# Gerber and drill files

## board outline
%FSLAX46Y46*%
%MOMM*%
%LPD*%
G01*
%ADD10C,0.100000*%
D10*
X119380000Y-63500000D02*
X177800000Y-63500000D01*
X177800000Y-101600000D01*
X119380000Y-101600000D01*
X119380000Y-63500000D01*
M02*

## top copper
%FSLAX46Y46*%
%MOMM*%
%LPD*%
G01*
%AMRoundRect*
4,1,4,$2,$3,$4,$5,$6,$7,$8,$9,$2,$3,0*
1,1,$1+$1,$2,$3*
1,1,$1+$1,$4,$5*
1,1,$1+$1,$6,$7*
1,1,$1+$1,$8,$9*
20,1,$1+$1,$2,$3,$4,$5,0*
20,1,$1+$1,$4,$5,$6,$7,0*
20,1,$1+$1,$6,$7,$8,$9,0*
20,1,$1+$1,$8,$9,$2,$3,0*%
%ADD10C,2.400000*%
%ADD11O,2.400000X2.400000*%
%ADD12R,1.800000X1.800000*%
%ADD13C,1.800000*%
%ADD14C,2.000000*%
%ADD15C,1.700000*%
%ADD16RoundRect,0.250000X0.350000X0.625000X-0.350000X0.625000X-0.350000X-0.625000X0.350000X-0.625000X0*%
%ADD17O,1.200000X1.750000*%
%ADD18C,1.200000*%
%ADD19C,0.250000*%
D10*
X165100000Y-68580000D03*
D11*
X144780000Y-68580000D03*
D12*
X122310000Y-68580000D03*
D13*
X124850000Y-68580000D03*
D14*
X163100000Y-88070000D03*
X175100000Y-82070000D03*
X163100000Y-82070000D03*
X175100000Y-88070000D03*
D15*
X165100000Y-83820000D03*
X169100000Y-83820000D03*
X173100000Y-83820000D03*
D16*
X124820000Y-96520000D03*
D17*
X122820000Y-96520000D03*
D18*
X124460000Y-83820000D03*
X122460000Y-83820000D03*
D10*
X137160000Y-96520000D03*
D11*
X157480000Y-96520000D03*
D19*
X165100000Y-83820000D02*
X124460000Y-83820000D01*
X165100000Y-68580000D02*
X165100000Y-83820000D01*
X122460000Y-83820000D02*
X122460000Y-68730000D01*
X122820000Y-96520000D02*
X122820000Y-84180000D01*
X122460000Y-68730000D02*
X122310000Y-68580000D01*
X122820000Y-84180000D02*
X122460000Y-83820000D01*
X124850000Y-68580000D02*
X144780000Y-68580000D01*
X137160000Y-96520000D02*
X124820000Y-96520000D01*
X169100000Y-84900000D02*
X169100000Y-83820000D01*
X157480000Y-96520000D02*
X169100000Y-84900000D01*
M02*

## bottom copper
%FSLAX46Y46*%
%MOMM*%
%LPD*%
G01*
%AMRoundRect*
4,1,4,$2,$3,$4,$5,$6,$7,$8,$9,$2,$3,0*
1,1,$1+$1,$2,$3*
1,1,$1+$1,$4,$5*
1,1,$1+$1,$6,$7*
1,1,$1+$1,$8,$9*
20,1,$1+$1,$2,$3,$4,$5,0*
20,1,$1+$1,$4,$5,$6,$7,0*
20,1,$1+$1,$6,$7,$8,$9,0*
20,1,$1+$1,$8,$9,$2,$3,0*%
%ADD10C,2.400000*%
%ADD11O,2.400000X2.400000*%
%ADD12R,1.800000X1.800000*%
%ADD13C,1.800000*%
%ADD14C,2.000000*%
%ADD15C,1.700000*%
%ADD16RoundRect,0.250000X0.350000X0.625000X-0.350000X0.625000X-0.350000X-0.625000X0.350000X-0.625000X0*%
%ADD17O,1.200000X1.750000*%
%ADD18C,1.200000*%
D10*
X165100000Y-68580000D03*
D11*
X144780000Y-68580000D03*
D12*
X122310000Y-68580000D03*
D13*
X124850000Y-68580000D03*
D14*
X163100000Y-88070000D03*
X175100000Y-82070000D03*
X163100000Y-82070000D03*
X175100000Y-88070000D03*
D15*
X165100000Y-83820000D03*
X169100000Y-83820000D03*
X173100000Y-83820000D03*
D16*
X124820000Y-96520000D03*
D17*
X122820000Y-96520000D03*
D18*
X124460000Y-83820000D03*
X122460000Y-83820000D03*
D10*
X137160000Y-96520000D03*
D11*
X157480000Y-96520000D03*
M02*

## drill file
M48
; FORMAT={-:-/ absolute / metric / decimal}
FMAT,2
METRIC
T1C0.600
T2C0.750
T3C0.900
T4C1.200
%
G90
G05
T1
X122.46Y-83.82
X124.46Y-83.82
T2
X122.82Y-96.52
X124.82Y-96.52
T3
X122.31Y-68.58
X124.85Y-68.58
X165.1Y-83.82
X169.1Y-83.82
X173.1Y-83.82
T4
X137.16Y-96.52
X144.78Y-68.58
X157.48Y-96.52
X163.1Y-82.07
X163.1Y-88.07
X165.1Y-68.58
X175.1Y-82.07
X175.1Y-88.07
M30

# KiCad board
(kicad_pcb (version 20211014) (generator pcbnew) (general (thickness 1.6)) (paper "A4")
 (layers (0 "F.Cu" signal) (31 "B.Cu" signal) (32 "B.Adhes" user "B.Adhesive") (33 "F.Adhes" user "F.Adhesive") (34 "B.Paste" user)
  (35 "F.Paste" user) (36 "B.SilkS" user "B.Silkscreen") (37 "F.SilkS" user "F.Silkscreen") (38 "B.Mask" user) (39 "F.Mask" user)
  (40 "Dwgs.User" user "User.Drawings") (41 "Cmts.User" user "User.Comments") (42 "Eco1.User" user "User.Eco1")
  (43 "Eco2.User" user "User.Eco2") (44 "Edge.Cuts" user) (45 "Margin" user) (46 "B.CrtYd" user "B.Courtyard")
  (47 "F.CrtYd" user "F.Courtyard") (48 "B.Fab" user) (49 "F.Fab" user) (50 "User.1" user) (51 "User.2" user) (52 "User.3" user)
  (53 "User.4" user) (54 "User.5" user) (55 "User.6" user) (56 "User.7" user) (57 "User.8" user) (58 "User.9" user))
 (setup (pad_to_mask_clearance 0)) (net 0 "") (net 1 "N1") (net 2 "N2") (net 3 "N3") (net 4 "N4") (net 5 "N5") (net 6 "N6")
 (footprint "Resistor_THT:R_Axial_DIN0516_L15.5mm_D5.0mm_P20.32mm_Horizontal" (layer "F.Cu") (at 165.1 68.58 180)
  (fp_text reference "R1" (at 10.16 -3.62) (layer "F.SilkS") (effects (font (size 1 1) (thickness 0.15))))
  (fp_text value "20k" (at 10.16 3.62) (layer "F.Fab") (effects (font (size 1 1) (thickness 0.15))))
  (pad "1" thru_hole circle (at 0 0 180) (size 2.4 2.4) (drill 1.2) (layers *.Cu *.Mask) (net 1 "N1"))
  (pad "2" thru_hole oval (at 20.32 0 180) (size 2.4 2.4) (drill 1.2) (layers *.Cu *.Mask) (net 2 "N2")))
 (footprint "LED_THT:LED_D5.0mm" (layer "F.Cu") (at 122.31 68.58)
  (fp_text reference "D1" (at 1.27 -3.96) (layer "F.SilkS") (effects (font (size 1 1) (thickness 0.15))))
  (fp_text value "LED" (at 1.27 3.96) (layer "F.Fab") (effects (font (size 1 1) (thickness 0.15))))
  (pad "1" thru_hole rect (at 0 0) (size 1.8 1.8) (drill 0.9) (layers *.Cu *.Mask) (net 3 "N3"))
  (pad "2" thru_hole circle (at 2.54 0) (size 1.8 1.8) (drill 0.9) (layers *.Cu *.Mask) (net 2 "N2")))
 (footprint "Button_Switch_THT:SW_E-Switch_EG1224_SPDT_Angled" (layer "F.Cu") (at 165.1 83.82)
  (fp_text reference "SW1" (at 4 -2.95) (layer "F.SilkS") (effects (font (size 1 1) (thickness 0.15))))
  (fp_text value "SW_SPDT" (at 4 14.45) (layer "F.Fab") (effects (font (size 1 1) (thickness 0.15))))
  (pad "" thru_hole circle (at -2 4.25) (size 2 2) (drill 1.2) (layers *.Cu *.Mask))
  (pad "" thru_hole circle (at 10 -1.75) (size 2 2) (drill 1.2) (layers *.Cu *.Mask))
  (pad "" thru_hole circle (at -2 -1.75) (size 2 2) (drill 1.2) (layers *.Cu *.Mask))
  (pad "" thru_hole circle (at 10 4.25) (size 2 2) (drill 1.2) (layers *.Cu *.Mask))
  (pad "1" thru_hole circle (at 0 0) (size 1.7 1.7) (drill 0.9) (layers *.Cu *.Mask) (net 1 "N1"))
  (pad "2" thru_hole circle (at 4 0) (size 1.7 1.7) (drill 0.9) (layers *.Cu *.Mask) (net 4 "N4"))
  (pad "3" thru_hole circle (at 8 0) (size 1.7 1.7) (drill 0.9) (layers *.Cu *.Mask) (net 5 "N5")))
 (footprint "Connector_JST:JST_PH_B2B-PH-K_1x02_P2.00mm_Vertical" (layer "F.Cu") (at 124.82 96.52 180)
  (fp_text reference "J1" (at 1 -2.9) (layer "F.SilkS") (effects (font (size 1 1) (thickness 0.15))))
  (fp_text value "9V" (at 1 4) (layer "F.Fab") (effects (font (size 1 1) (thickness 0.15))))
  (pad "1" thru_hole roundrect (at 0 0 180) (size 1.2 1.75) (drill 0.75) (layers *.Cu *.Mask) (roundrect_rratio 0.208333) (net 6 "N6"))
  (pad "2" thru_hole oval (at 2 0 180) (size 1.2 1.75) (drill 0.75) (layers *.Cu *.Mask) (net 3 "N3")))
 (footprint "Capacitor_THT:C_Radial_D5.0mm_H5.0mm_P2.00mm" (layer "F.Cu") (at 124.46 83.82 180)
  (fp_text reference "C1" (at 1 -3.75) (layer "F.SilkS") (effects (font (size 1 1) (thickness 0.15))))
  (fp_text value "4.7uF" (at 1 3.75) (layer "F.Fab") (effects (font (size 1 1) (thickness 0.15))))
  (pad "1" thru_hole circle (at 0 0 180) (size 1.2 1.2) (drill 0.6) (layers *.Cu *.Mask) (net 1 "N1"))
  (pad "2" thru_hole circle (at 2 0 180) (size 1.2 1.2) (drill 0.6) (layers *.Cu *.Mask) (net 3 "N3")))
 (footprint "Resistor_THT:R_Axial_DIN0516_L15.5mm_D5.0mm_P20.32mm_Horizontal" (layer "F.Cu") (at 137.16 96.52)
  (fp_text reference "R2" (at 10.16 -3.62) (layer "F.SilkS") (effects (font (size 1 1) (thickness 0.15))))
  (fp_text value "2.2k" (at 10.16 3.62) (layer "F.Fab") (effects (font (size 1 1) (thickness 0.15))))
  (pad "1" thru_hole circle (at 0 0) (size 2.4 2.4) (drill 1.2) (layers *.Cu *.Mask) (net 6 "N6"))
  (pad "2" thru_hole oval (at 20.32 0) (size 2.4 2.4) (drill 1.2) (layers *.Cu *.Mask) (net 4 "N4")))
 (gr_rect (start 119.38 101.6) (end 177.8 63.5) (layer "Edge.Cuts") (width 0.1) (fill none))
 (segment (start 165.1 83.82) (end 124.46 83.82) (width 0.25) (layer "F.Cu") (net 1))
 (segment (start 165.1 68.58) (end 165.1 83.82) (width 0.25) (layer "F.Cu") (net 1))
 (segment (start 122.46 83.82) (end 122.46 68.73) (width 0.25) (layer "F.Cu") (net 3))
 (segment (start 122.82 96.52) (end 122.82 84.18) (width 0.25) (layer "F.Cu") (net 3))
 (segment (start 122.46 68.73) (end 122.31 68.58) (width 0.25) (layer "F.Cu") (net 3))
 (segment (start 122.82 84.18) (end 122.46 83.82) (width 0.25) (layer "F.Cu") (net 3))
 (segment (start 124.85 68.58) (end 144.78 68.58) (width 0.25) (layer "F.Cu") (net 2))
 (segment (start 137.16 96.52) (end 124.82 96.52) (width 0.25) (layer "F.Cu") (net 6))
 (segment (start 169.1 84.9) (end 169.1 83.82) (width 0.25) (layer "F.Cu") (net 4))
 (segment (start 157.48 96.52) (end 169.1 84.9) (width 0.25) (layer "F.Cu") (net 4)))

